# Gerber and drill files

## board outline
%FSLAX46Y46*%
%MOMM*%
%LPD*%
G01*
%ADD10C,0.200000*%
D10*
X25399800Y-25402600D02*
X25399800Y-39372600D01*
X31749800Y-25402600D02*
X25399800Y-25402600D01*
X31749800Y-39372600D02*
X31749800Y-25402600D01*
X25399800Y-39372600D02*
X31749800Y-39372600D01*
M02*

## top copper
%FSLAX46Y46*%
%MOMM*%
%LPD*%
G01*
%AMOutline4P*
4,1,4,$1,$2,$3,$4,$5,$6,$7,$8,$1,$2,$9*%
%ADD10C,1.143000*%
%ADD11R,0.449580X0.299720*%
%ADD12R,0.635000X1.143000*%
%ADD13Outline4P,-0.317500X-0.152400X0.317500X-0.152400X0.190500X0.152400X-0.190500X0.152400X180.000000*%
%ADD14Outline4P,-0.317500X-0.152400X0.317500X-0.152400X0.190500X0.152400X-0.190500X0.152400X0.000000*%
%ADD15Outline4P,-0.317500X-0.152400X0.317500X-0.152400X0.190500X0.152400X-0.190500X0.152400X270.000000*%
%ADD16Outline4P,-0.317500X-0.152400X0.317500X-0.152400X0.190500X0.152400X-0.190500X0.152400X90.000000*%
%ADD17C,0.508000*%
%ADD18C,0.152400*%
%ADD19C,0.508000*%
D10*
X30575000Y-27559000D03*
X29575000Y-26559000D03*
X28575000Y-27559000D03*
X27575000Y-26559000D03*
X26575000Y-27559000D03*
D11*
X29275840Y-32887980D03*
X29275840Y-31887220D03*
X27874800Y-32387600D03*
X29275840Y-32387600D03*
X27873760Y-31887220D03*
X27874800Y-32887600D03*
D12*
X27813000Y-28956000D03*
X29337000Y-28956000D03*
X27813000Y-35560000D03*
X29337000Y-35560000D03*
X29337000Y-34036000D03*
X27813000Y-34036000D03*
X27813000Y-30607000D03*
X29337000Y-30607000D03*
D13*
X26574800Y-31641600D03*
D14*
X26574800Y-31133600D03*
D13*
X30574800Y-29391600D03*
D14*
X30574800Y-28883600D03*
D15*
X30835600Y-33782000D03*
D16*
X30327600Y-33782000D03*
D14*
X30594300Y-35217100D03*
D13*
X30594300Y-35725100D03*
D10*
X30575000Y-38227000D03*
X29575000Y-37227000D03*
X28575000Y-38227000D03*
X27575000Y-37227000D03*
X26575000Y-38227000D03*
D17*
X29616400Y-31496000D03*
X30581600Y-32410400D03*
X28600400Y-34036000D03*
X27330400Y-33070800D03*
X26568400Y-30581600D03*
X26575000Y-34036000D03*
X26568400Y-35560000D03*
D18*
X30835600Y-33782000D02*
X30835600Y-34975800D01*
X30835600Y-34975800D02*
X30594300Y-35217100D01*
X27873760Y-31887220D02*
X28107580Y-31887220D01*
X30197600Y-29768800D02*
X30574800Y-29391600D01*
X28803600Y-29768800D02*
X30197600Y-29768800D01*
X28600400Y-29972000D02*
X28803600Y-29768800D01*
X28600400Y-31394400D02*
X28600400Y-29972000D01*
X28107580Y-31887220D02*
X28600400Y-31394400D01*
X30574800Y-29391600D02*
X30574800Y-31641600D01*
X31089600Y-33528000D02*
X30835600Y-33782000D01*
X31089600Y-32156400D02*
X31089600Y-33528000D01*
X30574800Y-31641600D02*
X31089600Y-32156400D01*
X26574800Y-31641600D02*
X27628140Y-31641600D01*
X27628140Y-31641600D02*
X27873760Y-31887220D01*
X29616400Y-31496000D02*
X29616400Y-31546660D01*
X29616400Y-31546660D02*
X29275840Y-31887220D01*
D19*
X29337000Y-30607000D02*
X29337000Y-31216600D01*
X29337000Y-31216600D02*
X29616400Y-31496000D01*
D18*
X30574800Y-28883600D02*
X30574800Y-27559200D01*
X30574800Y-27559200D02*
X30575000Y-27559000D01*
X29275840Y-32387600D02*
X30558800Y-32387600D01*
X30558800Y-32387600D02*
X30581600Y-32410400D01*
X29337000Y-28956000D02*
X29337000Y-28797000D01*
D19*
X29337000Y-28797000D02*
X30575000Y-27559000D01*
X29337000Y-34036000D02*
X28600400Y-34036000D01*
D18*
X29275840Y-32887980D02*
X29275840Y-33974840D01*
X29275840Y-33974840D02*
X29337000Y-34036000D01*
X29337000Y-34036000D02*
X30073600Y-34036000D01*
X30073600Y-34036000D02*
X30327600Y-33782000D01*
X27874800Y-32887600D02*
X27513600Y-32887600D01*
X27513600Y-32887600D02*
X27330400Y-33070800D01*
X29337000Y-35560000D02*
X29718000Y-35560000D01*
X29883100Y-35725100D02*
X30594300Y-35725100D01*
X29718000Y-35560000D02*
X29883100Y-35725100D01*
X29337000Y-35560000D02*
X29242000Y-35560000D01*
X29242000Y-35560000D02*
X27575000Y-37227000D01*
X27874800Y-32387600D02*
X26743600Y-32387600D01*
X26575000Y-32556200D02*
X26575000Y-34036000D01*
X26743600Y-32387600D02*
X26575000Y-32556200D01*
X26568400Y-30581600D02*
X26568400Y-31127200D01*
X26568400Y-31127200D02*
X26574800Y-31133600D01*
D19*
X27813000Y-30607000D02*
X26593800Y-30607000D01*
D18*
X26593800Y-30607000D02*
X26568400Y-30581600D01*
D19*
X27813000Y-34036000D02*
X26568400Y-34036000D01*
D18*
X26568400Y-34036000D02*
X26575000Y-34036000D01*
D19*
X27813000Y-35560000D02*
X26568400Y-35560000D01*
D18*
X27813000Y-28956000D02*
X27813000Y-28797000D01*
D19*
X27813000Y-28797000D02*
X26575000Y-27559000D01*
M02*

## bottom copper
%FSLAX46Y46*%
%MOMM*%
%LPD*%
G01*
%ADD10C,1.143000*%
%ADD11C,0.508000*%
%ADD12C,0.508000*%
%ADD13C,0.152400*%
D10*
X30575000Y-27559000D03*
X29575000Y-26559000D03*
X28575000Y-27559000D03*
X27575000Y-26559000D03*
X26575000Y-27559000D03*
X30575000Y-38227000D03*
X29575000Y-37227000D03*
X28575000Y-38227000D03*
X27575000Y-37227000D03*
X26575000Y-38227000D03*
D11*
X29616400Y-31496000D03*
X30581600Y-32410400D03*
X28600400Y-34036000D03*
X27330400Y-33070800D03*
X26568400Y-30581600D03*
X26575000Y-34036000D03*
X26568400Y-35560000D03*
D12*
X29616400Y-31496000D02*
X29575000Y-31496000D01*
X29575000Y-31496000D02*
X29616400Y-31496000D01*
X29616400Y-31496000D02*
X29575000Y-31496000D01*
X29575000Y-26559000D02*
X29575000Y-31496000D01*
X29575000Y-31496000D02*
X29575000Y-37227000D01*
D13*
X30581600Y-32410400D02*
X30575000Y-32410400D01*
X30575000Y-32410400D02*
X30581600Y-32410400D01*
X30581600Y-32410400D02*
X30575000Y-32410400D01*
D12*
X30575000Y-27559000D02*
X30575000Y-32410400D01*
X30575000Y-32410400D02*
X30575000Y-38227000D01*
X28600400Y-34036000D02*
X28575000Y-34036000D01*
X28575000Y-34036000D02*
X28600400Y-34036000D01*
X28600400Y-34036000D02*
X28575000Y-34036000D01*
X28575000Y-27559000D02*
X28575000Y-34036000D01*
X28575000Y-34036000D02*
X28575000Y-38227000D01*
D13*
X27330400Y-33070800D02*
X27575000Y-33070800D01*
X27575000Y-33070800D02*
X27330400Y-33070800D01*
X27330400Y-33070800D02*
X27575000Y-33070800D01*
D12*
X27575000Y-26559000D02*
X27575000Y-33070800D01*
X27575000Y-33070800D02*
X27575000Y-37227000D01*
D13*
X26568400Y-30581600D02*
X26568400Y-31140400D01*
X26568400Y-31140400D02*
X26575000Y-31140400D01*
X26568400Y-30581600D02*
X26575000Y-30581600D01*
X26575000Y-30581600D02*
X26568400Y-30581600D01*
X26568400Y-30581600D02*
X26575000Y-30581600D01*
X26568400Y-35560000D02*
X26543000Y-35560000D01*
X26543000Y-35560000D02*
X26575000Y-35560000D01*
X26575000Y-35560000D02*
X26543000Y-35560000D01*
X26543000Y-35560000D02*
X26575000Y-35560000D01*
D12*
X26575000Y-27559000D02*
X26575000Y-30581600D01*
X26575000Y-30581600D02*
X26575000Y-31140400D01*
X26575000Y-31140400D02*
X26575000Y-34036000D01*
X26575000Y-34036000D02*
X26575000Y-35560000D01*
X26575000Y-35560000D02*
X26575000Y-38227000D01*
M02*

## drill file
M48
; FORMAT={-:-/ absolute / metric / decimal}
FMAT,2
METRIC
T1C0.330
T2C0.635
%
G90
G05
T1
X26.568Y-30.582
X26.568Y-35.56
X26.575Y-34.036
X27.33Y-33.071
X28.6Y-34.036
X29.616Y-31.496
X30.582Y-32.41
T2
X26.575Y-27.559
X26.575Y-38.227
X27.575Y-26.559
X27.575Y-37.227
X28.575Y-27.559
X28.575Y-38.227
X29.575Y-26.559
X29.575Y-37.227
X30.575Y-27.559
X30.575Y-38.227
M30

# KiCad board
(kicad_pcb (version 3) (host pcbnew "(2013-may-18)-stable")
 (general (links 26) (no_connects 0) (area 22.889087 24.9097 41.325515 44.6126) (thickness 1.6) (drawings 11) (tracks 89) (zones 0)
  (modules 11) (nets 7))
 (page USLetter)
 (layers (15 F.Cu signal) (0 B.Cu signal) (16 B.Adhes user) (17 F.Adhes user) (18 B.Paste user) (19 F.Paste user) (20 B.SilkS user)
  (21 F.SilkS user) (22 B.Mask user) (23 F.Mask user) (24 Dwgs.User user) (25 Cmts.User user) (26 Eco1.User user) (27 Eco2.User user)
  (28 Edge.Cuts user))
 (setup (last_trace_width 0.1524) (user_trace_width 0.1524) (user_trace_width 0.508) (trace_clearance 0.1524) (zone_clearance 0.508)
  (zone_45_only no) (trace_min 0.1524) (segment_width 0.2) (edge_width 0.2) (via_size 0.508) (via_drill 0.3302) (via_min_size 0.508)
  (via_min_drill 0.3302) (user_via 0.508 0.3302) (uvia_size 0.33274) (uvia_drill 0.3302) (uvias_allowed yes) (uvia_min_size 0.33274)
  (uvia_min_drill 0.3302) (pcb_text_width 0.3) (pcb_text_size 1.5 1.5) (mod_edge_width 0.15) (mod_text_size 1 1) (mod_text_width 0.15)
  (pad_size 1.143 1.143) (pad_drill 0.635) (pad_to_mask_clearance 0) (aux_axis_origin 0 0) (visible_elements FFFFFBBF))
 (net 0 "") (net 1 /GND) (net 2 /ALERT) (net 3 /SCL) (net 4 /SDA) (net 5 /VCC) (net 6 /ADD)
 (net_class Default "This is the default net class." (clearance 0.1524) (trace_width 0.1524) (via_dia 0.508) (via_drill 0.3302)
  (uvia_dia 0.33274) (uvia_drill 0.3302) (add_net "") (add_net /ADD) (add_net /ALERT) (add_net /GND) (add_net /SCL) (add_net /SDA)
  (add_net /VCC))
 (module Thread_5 (layer F.Cu) (at 28.575 27.559 180)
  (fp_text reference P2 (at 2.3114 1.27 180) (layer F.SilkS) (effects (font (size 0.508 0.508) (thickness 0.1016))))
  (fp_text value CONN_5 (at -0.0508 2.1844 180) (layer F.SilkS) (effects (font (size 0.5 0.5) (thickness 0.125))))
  (pad 1 thru_hole circle (at -2 0 180) (size 1.143 1.143) (drill 0.635) (layers *.Cu *.Mask F.SilkS) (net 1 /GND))
  (pad 2 thru_hole circle (at -1 1 180) (size 1.143 1.143) (drill 0.635) (layers *.Cu *.Mask F.SilkS) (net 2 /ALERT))
  (pad 3 thru_hole circle (at 0 0 180) (size 1.143 1.143) (drill 0.635) (layers *.Cu *.Mask F.SilkS) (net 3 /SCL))
  (pad 4 thru_hole circle (at 1 1 180) (size 1.143 1.143) (drill 0.635) (layers *.Cu *.Mask F.SilkS) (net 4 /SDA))
  (pad 5 thru_hole circle (at 2 0 180) (size 1.143 1.143) (drill 0.635) (layers *.Cu *.Mask F.SilkS) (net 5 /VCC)))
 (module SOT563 (layer F.Cu) (at 28.5748 32.3876 180)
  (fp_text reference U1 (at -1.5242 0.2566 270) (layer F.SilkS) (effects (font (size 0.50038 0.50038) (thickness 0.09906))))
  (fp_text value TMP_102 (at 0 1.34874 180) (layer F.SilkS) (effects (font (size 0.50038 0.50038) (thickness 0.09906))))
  (pad 1 smd rect (at -0.70104 -0.50038 180) (size 0.44958 0.29972) (layers F.Cu F.Paste F.Mask) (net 3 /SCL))
  (pad 3 smd rect (at -0.70104 0.50038 180) (size 0.44958 0.29972) (layers F.Cu F.Paste F.Mask) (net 2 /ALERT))
  (pad 5 smd rect (at 0.7 0 180) (size 0.44958 0.29972) (layers F.Cu F.Paste F.Mask) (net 5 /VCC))
  (pad 2 smd rect (at -0.70104 0 180) (size 0.44958 0.29972) (layers F.Cu F.Paste F.Mask) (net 1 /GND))
  (pad 4 smd rect (at 0.70104 0.50038 180) (size 0.44958 0.29972) (layers F.Cu F.Paste F.Mask) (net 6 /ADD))
  (pad 6 smd rect (at 0.7 -0.5 180) (size 0.44958 0.29972) (layers F.Cu F.Paste F.Mask) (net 4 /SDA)))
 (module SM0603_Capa (layer F.Cu) (at 28.575 28.956)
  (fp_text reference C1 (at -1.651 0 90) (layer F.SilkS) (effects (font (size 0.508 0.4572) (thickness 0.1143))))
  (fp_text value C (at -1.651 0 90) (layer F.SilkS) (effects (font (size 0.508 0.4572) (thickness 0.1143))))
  (pad 1 smd rect (at -0.762 0) (size 0.635 1.143) (layers F.Cu F.Paste F.Mask) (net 5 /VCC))
  (pad 2 smd rect (at 0.762 0) (size 0.635 1.143) (layers F.Cu F.Paste F.Mask) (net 1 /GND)))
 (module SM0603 (layer F.Cu) (at 28.575 35.56)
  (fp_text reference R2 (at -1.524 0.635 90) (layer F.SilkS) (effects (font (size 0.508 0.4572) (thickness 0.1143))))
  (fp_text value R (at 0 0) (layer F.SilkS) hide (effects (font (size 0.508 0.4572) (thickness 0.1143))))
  (pad 1 smd rect (at -0.762 0) (size 0.635 1.143) (layers F.Cu F.Paste F.Mask) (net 5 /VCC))
  (pad 2 smd rect (at 0.762 0) (size 0.635 1.143) (layers F.Cu F.Paste F.Mask) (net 4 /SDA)))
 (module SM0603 (layer F.Cu) (at 28.575 34.036 180)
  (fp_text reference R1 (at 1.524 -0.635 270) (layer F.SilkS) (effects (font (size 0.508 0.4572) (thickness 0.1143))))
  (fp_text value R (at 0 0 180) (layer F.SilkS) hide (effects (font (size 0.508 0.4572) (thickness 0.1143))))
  (pad 1 smd rect (at -0.762 0 180) (size 0.635 1.143) (layers F.Cu F.Paste F.Mask) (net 5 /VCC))
  (pad 2 smd rect (at 0.762 0 180) (size 0.635 1.143) (layers F.Cu F.Paste F.Mask) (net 3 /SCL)))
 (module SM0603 (layer F.Cu) (at 28.575 30.607)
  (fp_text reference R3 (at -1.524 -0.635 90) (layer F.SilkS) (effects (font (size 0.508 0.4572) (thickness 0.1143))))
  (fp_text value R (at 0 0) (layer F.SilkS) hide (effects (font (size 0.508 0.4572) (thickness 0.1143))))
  (pad 1 smd rect (at -0.762 0) (size 0.635 1.143) (layers F.Cu F.Paste F.Mask) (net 5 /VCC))
  (pad 2 smd rect (at 0.762 0) (size 0.635 1.143) (layers F.Cu F.Paste F.Mask) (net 2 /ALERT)))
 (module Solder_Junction (layer F.Cu) (at 26.5748 31.3876 90)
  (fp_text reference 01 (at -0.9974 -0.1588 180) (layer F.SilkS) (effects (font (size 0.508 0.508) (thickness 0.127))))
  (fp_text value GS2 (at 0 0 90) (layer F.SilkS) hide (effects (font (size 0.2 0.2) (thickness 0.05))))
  (pad 1 smd trapezoid (at -0.254 0 180) (size 0.508 0.3048) (rect_delta 0 0.127) (layers F.Cu F.Paste F.Mask) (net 6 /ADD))
  (pad 2 smd trapezoid (at 0.254 0) (size 0.508 0.3048) (rect_delta 0 0.127) (layers F.Cu F.Paste F.Mask) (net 5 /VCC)))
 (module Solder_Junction (layer F.Cu) (at 30.5748 29.1376 90)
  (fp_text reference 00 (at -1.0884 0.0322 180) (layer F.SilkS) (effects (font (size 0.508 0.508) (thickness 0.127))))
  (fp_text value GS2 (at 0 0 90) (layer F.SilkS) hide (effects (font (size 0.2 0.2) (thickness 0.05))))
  (pad 1 smd trapezoid (at -0.254 0 180) (size 0.508 0.3048) (rect_delta 0 0.127) (layers F.Cu F.Paste F.Mask) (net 6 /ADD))
  (pad 2 smd trapezoid (at 0.254 0) (size 0.508 0.3048) (rect_delta 0 0.127) (layers F.Cu F.Paste F.Mask) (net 1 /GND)))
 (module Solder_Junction (layer F.Cu) (at 30.5816 33.782 180)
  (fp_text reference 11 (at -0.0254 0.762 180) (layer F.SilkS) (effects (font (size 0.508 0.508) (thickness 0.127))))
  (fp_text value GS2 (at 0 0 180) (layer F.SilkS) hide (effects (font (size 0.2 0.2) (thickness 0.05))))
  (pad 1 smd trapezoid (at -0.254 0 270) (size 0.508 0.3048) (rect_delta 0 0.127) (layers F.Cu F.Paste F.Mask) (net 6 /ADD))
  (pad 2 smd trapezoid (at 0.254 0 90) (size 0.508 0.3048) (rect_delta 0 0.127) (layers F.Cu F.Paste F.Mask) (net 3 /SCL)))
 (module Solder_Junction (layer F.Cu) (at 30.5943 35.4711 270)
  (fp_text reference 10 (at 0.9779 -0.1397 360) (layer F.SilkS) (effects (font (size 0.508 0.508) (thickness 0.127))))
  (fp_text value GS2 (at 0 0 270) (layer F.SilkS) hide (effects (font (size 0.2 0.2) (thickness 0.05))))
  (pad 1 smd trapezoid (at -0.254 0) (size 0.508 0.3048) (rect_delta 0 0.127) (layers F.Cu F.Paste F.Mask) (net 6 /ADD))
  (pad 2 smd trapezoid (at 0.254 0 180) (size 0.508 0.3048) (rect_delta 0 0.127) (layers F.Cu F.Paste F.Mask) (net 4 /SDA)))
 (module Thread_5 (layer F.Cu) (at 28.575 38.227 180)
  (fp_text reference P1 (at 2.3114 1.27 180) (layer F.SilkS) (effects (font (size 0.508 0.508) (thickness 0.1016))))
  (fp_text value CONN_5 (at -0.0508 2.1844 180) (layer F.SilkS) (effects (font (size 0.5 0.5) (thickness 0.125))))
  (pad 1 thru_hole circle (at -2 0 180) (size 1.143 1.143) (drill 0.635) (layers *.Cu *.Mask F.SilkS) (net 1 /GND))
  (pad 2 thru_hole circle (at -1 1 180) (size 1.143 1.143) (drill 0.635) (layers *.Cu *.Mask F.SilkS) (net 2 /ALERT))
  (pad 3 thru_hole circle (at 0 0 180) (size 1.143 1.143) (drill 0.635) (layers *.Cu *.Mask F.SilkS) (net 3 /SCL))
  (pad 4 thru_hole circle (at 1 1 180) (size 1.143 1.143) (drill 0.635) (layers *.Cu *.Mask F.SilkS) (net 4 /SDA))
  (pad 5 thru_hole circle (at 2 0 180) (size 1.143 1.143) (drill 0.635) (layers *.Cu *.Mask F.SilkS) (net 5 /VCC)))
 (gr_line (start 25.3998 25.4026) (end 25.3998 39.3726) (angle 90) (layer Edge.Cuts) (width 0.2))
 (gr_line (start 31.7498 25.4026) (end 25.3998 25.4026) (angle 90) (layer Edge.Cuts) (width 0.2))
 (gr_line (start 31.7498 39.3726) (end 31.7498 25.4026) (angle 90) (layer Edge.Cuts) (width 0.2))
 (gr_line (start 25.3998 39.3726) (end 31.7498 39.3726) (angle 90) (layer Edge.Cuts) (width 0.2))
 (segment (start 30.8356 33.782) (end 30.8356 34.9758) (width 0.1524) (layer F.Cu) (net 6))
 (segment (start 30.8356 34.9758) (end 30.5943 35.2171) (width 0.1524) (layer F.Cu) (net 6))
 (segment (start 27.87376 31.88722) (end 28.10758 31.88722) (width 0.1524) (layer F.Cu) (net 6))
 (segment (start 30.1976 29.7688) (end 30.5748 29.3916) (width 0.1524) (layer F.Cu) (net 6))
 (segment (start 28.8036 29.7688) (end 30.1976 29.7688) (width 0.1524) (layer F.Cu) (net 6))
 (segment (start 28.6004 29.972) (end 28.8036 29.7688) (width 0.1524) (layer F.Cu) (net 6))
 (segment (start 28.6004 31.3944) (end 28.6004 29.972) (width 0.1524) (layer F.Cu) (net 6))
 (segment (start 28.10758 31.88722) (end 28.6004 31.3944) (width 0.1524) (layer F.Cu) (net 6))
 (segment (start 30.5748 29.3916) (end 30.5748 31.6416) (width 0.1524) (layer F.Cu) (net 6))
 (segment (start 31.0896 33.528) (end 30.8356 33.782) (width 0.1524) (layer F.Cu) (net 6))
 (segment (start 31.0896 32.1564) (end 31.0896 33.528) (width 0.1524) (layer F.Cu) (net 6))
 (segment (start 30.5748 31.6416) (end 31.0896 32.1564) (width 0.1524) (layer F.Cu) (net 6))
 (segment (start 26.5748 31.6416) (end 27.62814 31.6416) (width 0.1524) (layer F.Cu) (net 6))
 (segment (start 27.62814 31.6416) (end 27.87376 31.88722) (width 0.1524) (layer F.Cu) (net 6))
 (segment (start 29.6164 31.496) (end 29.6164 31.54666) (width 0.1524) (layer F.Cu) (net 2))
 (segment (start 29.6164 31.54666) (end 29.27584 31.88722) (width 0.1524) (layer F.Cu) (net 2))
 (segment (start 29.337 30.607) (end 29.337 31.2166) (width 0.508) (layer F.Cu) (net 2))
 (via (at 29.6164 31.496) (size 0.508) (layers F.Cu B.Cu) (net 2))
 (segment (start 29.337 31.2166) (end 29.6164 31.496) (width 0.508) (layer F.Cu) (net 2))
 (segment (start 29.6164 31.496) (end 29.575 31.496) (width 0.508) (layer B.Cu) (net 2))
 (segment (start 29.575 31.496) (end 29.6164 31.496) (width 0.508) (layer B.Cu) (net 2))
 (segment (start 29.6164 31.496) (end 29.575 31.496) (width 0.508) (layer B.Cu) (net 2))
 (segment (start 29.575 26.559) (end 29.575 31.496) (width 0.508) (layer B.Cu) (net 2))
 (segment (start 29.575 31.496) (end 29.575 37.227) (width 0.508) (layer B.Cu) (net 2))
 (segment (start 30.5748 28.8836) (end 30.5748 27.5592) (width 0.1524) (layer F.Cu) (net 1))
 (segment (start 30.5748 27.5592) (end 30.575 27.559) (width 0.1524) (layer F.Cu) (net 1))
 (segment (start 29.27584 32.3876) (end 30.5588 32.3876) (width 0.1524) (layer F.Cu) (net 1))
 (via (at 30.5816 32.4104) (size 0.508) (layers F.Cu B.Cu) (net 1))
 (segment (start 30.5588 32.3876) (end 30.5816 32.4104) (width 0.1524) (layer F.Cu) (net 1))
 (segment (start 30.5816 32.4104) (end 30.575 32.4104) (width 0.1524) (layer B.Cu) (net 1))
 (segment (start 30.575 32.4104) (end 30.5816 32.4104) (width 0.1524) (layer B.Cu) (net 1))
 (segment (start 30.5816 32.4104) (end 30.575 32.4104) (width 0.1524) (layer B.Cu) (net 1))
 (segment (start 29.337 28.956) (end 29.337 28.797) (width 0.1524) (layer F.Cu) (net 1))
 (segment (start 29.337 28.797) (end 30.575 27.559) (width 0.508) (layer F.Cu) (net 1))
 (segment (start 30.575 27.559) (end 30.575 32.4104) (width 0.508) (layer B.Cu) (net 1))
 (segment (start 30.575 32.4104) (end 30.575 38.227) (width 0.508) (layer B.Cu) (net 1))
 (segment (start 29.337 34.036) (end 28.6004 34.036) (width 0.508) (layer F.Cu) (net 3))
 (via (at 28.6004 34.036) (size 0.508) (layers F.Cu B.Cu) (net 3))
 (segment (start 28.6004 34.036) (end 28.575 34.036) (width 0.508) (layer B.Cu) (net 3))
 (segment (start 28.575 34.036) (end 28.6004 34.036) (width 0.508) (layer B.Cu) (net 3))
 (segment (start 28.6004 34.036) (end 28.575 34.036) (width 0.508) (layer B.Cu) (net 3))
 (segment (start 29.27584 32.88798) (end 29.27584 33.97484) (width 0.1524) (layer F.Cu) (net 3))
 (segment (start 29.27584 33.97484) (end 29.337 34.036) (width 0.1524) (layer F.Cu) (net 3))
 (segment (start 29.337 34.036) (end 30.0736 34.036) (width 0.1524) (layer F.Cu) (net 3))
 (segment (start 30.0736 34.036) (end 30.3276 33.782) (width 0.1524) (layer F.Cu) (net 3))
 (segment (start 28.575 27.559) (end 28.575 34.036) (width 0.508) (layer B.Cu) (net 3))
 (segment (start 28.575 34.036) (end 28.575 38.227) (width 0.508) (layer B.Cu) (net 3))
 (segment (start 27.8748 32.8876) (end 27.5136 32.8876) (width 0.1524) (layer F.Cu) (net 4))
 (via (at 27.3304 33.0708) (size 0.508) (layers F.Cu B.Cu) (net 4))
 (segment (start 27.5136 32.8876) (end 27.3304 33.0708) (width 0.1524) (layer F.Cu) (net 4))
 (segment (start 27.3304 33.0708) (end 27.575 33.0708) (width 0.1524) (layer B.Cu) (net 4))
 (segment (start 27.575 33.0708) (end 27.3304 33.0708) (width 0.1524) (layer B.Cu) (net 4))
 (segment (start 27.3304 33.0708) (end 27.575 33.0708) (width 0.1524) (layer B.Cu) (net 4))
 (segment (start 29.337 35.56) (end 29.718 35.56) (width 0.1524) (layer F.Cu) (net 4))
 (segment (start 29.8831 35.7251) (end 30.5943 35.7251) (width 0.1524) (layer F.Cu) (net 4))
 (segment (start 29.718 35.56) (end 29.8831 35.7251) (width 0.1524) (layer F.Cu) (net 4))
 (segment (start 29.337 35.56) (end 29.242 35.56) (width 0.1524) (layer F.Cu) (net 4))
 (segment (start 29.242 35.56) (end 27.575 37.227) (width 0.1524) (layer F.Cu) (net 4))
 (segment (start 27.575 26.559) (end 27.575 33.0708) (width 0.508) (layer B.Cu) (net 4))
 (segment (start 27.575 33.0708) (end 27.575 37.227) (width 0.508) (layer B.Cu) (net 4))
 (segment (start 27.8748 32.3876) (end 26.7436 32.3876) (width 0.1524) (layer F.Cu) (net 5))
 (segment (start 26.575 32.5562) (end 26.575 34.036) (width 0.1524) (layer F.Cu) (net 5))
 (segment (start 26.7436 32.3876) (end 26.575 32.5562) (width 0.1524) (layer F.Cu) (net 5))
 (segment (start 26.5684 30.5816) (end 26.5684 31.1272) (width 0.1524) (layer F.Cu) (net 5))
 (segment (start 26.5684 31.1272) (end 26.5748 31.1336) (width 0.1524) (layer F.Cu) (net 5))
 (segment (start 26.5684 30.5816) (end 26.5684 31.1404) (width 0.1524) (layer B.Cu) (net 5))
 (segment (start 26.5684 31.1404) (end 26.575 31.1404) (width 0.1524) (layer B.Cu) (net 5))
 (segment (start 27.813 30.607) (end 26.5938 30.607) (width 0.508) (layer F.Cu) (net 5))
 (via (at 26.5684 30.5816) (size 0.508) (layers F.Cu B.Cu) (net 5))
 (segment (start 26.5938 30.607) (end 26.5684 30.5816) (width 0.1524) (layer F.Cu) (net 5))
 (segment (start 26.5684 30.5816) (end 26.575 30.5816) (width 0.1524) (layer B.Cu) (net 5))
 (segment (start 26.575 30.5816) (end 26.5684 30.5816) (width 0.1524) (layer B.Cu) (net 5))
 (segment (start 26.5684 30.5816) (end 26.575 30.5816) (width 0.1524) (layer B.Cu) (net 5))
 (via (at 26.575 34.036) (size 0.508) (layers F.Cu B.Cu) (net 5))
 (segment (start 27.813 34.036) (end 26.5684 34.036) (width 0.508) (layer F.Cu) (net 5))
 (segment (start 26.5684 34.036) (end 26.575 34.036) (width 0.1524) (layer F.Cu) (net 5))
 (segment (start 27.813 35.56) (end 26.5684 35.56) (width 0.508) (layer F.Cu) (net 5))
 (segment (start 26.5684 35.56) (end 26.543 35.56) (width 0.1524) (layer B.Cu) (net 5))
 (via (at 26.5684 35.56) (size 0.508) (layers F.Cu B.Cu) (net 5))
 (segment (start 26.543 35.56) (end 26.575 35.56) (width 0.1524) (layer B.Cu) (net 5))
 (segment (start 26.575 35.56) (end 26.543 35.56) (width 0.1524) (layer B.Cu) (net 5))
 (segment (start 26.543 35.56) (end 26.575 35.56) (width 0.1524) (layer B.Cu) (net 5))
 (segment (start 27.813 28.956) (end 27.813 28.797) (width 0.1524) (layer F.Cu) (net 5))
 (segment (start 27.813 28.797) (end 26.575 27.559) (width 0.508) (layer F.Cu) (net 5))
 (segment (start 26.575 27.559) (end 26.575 30.5816) (width 0.508) (layer B.Cu) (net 5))
 (segment (start 26.575 30.5816) (end 26.575 31.1404) (width 0.508) (layer B.Cu) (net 5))
 (segment (start 26.575 31.1404) (end 26.575 34.036) (width 0.508) (layer B.Cu) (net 5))
 (segment (start 26.575 34.036) (end 26.575 35.56) (width 0.508) (layer B.Cu) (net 5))
 (segment (start 26.575 35.56) (end 26.575 38.227) (width 0.508) (layer B.Cu) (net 5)))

